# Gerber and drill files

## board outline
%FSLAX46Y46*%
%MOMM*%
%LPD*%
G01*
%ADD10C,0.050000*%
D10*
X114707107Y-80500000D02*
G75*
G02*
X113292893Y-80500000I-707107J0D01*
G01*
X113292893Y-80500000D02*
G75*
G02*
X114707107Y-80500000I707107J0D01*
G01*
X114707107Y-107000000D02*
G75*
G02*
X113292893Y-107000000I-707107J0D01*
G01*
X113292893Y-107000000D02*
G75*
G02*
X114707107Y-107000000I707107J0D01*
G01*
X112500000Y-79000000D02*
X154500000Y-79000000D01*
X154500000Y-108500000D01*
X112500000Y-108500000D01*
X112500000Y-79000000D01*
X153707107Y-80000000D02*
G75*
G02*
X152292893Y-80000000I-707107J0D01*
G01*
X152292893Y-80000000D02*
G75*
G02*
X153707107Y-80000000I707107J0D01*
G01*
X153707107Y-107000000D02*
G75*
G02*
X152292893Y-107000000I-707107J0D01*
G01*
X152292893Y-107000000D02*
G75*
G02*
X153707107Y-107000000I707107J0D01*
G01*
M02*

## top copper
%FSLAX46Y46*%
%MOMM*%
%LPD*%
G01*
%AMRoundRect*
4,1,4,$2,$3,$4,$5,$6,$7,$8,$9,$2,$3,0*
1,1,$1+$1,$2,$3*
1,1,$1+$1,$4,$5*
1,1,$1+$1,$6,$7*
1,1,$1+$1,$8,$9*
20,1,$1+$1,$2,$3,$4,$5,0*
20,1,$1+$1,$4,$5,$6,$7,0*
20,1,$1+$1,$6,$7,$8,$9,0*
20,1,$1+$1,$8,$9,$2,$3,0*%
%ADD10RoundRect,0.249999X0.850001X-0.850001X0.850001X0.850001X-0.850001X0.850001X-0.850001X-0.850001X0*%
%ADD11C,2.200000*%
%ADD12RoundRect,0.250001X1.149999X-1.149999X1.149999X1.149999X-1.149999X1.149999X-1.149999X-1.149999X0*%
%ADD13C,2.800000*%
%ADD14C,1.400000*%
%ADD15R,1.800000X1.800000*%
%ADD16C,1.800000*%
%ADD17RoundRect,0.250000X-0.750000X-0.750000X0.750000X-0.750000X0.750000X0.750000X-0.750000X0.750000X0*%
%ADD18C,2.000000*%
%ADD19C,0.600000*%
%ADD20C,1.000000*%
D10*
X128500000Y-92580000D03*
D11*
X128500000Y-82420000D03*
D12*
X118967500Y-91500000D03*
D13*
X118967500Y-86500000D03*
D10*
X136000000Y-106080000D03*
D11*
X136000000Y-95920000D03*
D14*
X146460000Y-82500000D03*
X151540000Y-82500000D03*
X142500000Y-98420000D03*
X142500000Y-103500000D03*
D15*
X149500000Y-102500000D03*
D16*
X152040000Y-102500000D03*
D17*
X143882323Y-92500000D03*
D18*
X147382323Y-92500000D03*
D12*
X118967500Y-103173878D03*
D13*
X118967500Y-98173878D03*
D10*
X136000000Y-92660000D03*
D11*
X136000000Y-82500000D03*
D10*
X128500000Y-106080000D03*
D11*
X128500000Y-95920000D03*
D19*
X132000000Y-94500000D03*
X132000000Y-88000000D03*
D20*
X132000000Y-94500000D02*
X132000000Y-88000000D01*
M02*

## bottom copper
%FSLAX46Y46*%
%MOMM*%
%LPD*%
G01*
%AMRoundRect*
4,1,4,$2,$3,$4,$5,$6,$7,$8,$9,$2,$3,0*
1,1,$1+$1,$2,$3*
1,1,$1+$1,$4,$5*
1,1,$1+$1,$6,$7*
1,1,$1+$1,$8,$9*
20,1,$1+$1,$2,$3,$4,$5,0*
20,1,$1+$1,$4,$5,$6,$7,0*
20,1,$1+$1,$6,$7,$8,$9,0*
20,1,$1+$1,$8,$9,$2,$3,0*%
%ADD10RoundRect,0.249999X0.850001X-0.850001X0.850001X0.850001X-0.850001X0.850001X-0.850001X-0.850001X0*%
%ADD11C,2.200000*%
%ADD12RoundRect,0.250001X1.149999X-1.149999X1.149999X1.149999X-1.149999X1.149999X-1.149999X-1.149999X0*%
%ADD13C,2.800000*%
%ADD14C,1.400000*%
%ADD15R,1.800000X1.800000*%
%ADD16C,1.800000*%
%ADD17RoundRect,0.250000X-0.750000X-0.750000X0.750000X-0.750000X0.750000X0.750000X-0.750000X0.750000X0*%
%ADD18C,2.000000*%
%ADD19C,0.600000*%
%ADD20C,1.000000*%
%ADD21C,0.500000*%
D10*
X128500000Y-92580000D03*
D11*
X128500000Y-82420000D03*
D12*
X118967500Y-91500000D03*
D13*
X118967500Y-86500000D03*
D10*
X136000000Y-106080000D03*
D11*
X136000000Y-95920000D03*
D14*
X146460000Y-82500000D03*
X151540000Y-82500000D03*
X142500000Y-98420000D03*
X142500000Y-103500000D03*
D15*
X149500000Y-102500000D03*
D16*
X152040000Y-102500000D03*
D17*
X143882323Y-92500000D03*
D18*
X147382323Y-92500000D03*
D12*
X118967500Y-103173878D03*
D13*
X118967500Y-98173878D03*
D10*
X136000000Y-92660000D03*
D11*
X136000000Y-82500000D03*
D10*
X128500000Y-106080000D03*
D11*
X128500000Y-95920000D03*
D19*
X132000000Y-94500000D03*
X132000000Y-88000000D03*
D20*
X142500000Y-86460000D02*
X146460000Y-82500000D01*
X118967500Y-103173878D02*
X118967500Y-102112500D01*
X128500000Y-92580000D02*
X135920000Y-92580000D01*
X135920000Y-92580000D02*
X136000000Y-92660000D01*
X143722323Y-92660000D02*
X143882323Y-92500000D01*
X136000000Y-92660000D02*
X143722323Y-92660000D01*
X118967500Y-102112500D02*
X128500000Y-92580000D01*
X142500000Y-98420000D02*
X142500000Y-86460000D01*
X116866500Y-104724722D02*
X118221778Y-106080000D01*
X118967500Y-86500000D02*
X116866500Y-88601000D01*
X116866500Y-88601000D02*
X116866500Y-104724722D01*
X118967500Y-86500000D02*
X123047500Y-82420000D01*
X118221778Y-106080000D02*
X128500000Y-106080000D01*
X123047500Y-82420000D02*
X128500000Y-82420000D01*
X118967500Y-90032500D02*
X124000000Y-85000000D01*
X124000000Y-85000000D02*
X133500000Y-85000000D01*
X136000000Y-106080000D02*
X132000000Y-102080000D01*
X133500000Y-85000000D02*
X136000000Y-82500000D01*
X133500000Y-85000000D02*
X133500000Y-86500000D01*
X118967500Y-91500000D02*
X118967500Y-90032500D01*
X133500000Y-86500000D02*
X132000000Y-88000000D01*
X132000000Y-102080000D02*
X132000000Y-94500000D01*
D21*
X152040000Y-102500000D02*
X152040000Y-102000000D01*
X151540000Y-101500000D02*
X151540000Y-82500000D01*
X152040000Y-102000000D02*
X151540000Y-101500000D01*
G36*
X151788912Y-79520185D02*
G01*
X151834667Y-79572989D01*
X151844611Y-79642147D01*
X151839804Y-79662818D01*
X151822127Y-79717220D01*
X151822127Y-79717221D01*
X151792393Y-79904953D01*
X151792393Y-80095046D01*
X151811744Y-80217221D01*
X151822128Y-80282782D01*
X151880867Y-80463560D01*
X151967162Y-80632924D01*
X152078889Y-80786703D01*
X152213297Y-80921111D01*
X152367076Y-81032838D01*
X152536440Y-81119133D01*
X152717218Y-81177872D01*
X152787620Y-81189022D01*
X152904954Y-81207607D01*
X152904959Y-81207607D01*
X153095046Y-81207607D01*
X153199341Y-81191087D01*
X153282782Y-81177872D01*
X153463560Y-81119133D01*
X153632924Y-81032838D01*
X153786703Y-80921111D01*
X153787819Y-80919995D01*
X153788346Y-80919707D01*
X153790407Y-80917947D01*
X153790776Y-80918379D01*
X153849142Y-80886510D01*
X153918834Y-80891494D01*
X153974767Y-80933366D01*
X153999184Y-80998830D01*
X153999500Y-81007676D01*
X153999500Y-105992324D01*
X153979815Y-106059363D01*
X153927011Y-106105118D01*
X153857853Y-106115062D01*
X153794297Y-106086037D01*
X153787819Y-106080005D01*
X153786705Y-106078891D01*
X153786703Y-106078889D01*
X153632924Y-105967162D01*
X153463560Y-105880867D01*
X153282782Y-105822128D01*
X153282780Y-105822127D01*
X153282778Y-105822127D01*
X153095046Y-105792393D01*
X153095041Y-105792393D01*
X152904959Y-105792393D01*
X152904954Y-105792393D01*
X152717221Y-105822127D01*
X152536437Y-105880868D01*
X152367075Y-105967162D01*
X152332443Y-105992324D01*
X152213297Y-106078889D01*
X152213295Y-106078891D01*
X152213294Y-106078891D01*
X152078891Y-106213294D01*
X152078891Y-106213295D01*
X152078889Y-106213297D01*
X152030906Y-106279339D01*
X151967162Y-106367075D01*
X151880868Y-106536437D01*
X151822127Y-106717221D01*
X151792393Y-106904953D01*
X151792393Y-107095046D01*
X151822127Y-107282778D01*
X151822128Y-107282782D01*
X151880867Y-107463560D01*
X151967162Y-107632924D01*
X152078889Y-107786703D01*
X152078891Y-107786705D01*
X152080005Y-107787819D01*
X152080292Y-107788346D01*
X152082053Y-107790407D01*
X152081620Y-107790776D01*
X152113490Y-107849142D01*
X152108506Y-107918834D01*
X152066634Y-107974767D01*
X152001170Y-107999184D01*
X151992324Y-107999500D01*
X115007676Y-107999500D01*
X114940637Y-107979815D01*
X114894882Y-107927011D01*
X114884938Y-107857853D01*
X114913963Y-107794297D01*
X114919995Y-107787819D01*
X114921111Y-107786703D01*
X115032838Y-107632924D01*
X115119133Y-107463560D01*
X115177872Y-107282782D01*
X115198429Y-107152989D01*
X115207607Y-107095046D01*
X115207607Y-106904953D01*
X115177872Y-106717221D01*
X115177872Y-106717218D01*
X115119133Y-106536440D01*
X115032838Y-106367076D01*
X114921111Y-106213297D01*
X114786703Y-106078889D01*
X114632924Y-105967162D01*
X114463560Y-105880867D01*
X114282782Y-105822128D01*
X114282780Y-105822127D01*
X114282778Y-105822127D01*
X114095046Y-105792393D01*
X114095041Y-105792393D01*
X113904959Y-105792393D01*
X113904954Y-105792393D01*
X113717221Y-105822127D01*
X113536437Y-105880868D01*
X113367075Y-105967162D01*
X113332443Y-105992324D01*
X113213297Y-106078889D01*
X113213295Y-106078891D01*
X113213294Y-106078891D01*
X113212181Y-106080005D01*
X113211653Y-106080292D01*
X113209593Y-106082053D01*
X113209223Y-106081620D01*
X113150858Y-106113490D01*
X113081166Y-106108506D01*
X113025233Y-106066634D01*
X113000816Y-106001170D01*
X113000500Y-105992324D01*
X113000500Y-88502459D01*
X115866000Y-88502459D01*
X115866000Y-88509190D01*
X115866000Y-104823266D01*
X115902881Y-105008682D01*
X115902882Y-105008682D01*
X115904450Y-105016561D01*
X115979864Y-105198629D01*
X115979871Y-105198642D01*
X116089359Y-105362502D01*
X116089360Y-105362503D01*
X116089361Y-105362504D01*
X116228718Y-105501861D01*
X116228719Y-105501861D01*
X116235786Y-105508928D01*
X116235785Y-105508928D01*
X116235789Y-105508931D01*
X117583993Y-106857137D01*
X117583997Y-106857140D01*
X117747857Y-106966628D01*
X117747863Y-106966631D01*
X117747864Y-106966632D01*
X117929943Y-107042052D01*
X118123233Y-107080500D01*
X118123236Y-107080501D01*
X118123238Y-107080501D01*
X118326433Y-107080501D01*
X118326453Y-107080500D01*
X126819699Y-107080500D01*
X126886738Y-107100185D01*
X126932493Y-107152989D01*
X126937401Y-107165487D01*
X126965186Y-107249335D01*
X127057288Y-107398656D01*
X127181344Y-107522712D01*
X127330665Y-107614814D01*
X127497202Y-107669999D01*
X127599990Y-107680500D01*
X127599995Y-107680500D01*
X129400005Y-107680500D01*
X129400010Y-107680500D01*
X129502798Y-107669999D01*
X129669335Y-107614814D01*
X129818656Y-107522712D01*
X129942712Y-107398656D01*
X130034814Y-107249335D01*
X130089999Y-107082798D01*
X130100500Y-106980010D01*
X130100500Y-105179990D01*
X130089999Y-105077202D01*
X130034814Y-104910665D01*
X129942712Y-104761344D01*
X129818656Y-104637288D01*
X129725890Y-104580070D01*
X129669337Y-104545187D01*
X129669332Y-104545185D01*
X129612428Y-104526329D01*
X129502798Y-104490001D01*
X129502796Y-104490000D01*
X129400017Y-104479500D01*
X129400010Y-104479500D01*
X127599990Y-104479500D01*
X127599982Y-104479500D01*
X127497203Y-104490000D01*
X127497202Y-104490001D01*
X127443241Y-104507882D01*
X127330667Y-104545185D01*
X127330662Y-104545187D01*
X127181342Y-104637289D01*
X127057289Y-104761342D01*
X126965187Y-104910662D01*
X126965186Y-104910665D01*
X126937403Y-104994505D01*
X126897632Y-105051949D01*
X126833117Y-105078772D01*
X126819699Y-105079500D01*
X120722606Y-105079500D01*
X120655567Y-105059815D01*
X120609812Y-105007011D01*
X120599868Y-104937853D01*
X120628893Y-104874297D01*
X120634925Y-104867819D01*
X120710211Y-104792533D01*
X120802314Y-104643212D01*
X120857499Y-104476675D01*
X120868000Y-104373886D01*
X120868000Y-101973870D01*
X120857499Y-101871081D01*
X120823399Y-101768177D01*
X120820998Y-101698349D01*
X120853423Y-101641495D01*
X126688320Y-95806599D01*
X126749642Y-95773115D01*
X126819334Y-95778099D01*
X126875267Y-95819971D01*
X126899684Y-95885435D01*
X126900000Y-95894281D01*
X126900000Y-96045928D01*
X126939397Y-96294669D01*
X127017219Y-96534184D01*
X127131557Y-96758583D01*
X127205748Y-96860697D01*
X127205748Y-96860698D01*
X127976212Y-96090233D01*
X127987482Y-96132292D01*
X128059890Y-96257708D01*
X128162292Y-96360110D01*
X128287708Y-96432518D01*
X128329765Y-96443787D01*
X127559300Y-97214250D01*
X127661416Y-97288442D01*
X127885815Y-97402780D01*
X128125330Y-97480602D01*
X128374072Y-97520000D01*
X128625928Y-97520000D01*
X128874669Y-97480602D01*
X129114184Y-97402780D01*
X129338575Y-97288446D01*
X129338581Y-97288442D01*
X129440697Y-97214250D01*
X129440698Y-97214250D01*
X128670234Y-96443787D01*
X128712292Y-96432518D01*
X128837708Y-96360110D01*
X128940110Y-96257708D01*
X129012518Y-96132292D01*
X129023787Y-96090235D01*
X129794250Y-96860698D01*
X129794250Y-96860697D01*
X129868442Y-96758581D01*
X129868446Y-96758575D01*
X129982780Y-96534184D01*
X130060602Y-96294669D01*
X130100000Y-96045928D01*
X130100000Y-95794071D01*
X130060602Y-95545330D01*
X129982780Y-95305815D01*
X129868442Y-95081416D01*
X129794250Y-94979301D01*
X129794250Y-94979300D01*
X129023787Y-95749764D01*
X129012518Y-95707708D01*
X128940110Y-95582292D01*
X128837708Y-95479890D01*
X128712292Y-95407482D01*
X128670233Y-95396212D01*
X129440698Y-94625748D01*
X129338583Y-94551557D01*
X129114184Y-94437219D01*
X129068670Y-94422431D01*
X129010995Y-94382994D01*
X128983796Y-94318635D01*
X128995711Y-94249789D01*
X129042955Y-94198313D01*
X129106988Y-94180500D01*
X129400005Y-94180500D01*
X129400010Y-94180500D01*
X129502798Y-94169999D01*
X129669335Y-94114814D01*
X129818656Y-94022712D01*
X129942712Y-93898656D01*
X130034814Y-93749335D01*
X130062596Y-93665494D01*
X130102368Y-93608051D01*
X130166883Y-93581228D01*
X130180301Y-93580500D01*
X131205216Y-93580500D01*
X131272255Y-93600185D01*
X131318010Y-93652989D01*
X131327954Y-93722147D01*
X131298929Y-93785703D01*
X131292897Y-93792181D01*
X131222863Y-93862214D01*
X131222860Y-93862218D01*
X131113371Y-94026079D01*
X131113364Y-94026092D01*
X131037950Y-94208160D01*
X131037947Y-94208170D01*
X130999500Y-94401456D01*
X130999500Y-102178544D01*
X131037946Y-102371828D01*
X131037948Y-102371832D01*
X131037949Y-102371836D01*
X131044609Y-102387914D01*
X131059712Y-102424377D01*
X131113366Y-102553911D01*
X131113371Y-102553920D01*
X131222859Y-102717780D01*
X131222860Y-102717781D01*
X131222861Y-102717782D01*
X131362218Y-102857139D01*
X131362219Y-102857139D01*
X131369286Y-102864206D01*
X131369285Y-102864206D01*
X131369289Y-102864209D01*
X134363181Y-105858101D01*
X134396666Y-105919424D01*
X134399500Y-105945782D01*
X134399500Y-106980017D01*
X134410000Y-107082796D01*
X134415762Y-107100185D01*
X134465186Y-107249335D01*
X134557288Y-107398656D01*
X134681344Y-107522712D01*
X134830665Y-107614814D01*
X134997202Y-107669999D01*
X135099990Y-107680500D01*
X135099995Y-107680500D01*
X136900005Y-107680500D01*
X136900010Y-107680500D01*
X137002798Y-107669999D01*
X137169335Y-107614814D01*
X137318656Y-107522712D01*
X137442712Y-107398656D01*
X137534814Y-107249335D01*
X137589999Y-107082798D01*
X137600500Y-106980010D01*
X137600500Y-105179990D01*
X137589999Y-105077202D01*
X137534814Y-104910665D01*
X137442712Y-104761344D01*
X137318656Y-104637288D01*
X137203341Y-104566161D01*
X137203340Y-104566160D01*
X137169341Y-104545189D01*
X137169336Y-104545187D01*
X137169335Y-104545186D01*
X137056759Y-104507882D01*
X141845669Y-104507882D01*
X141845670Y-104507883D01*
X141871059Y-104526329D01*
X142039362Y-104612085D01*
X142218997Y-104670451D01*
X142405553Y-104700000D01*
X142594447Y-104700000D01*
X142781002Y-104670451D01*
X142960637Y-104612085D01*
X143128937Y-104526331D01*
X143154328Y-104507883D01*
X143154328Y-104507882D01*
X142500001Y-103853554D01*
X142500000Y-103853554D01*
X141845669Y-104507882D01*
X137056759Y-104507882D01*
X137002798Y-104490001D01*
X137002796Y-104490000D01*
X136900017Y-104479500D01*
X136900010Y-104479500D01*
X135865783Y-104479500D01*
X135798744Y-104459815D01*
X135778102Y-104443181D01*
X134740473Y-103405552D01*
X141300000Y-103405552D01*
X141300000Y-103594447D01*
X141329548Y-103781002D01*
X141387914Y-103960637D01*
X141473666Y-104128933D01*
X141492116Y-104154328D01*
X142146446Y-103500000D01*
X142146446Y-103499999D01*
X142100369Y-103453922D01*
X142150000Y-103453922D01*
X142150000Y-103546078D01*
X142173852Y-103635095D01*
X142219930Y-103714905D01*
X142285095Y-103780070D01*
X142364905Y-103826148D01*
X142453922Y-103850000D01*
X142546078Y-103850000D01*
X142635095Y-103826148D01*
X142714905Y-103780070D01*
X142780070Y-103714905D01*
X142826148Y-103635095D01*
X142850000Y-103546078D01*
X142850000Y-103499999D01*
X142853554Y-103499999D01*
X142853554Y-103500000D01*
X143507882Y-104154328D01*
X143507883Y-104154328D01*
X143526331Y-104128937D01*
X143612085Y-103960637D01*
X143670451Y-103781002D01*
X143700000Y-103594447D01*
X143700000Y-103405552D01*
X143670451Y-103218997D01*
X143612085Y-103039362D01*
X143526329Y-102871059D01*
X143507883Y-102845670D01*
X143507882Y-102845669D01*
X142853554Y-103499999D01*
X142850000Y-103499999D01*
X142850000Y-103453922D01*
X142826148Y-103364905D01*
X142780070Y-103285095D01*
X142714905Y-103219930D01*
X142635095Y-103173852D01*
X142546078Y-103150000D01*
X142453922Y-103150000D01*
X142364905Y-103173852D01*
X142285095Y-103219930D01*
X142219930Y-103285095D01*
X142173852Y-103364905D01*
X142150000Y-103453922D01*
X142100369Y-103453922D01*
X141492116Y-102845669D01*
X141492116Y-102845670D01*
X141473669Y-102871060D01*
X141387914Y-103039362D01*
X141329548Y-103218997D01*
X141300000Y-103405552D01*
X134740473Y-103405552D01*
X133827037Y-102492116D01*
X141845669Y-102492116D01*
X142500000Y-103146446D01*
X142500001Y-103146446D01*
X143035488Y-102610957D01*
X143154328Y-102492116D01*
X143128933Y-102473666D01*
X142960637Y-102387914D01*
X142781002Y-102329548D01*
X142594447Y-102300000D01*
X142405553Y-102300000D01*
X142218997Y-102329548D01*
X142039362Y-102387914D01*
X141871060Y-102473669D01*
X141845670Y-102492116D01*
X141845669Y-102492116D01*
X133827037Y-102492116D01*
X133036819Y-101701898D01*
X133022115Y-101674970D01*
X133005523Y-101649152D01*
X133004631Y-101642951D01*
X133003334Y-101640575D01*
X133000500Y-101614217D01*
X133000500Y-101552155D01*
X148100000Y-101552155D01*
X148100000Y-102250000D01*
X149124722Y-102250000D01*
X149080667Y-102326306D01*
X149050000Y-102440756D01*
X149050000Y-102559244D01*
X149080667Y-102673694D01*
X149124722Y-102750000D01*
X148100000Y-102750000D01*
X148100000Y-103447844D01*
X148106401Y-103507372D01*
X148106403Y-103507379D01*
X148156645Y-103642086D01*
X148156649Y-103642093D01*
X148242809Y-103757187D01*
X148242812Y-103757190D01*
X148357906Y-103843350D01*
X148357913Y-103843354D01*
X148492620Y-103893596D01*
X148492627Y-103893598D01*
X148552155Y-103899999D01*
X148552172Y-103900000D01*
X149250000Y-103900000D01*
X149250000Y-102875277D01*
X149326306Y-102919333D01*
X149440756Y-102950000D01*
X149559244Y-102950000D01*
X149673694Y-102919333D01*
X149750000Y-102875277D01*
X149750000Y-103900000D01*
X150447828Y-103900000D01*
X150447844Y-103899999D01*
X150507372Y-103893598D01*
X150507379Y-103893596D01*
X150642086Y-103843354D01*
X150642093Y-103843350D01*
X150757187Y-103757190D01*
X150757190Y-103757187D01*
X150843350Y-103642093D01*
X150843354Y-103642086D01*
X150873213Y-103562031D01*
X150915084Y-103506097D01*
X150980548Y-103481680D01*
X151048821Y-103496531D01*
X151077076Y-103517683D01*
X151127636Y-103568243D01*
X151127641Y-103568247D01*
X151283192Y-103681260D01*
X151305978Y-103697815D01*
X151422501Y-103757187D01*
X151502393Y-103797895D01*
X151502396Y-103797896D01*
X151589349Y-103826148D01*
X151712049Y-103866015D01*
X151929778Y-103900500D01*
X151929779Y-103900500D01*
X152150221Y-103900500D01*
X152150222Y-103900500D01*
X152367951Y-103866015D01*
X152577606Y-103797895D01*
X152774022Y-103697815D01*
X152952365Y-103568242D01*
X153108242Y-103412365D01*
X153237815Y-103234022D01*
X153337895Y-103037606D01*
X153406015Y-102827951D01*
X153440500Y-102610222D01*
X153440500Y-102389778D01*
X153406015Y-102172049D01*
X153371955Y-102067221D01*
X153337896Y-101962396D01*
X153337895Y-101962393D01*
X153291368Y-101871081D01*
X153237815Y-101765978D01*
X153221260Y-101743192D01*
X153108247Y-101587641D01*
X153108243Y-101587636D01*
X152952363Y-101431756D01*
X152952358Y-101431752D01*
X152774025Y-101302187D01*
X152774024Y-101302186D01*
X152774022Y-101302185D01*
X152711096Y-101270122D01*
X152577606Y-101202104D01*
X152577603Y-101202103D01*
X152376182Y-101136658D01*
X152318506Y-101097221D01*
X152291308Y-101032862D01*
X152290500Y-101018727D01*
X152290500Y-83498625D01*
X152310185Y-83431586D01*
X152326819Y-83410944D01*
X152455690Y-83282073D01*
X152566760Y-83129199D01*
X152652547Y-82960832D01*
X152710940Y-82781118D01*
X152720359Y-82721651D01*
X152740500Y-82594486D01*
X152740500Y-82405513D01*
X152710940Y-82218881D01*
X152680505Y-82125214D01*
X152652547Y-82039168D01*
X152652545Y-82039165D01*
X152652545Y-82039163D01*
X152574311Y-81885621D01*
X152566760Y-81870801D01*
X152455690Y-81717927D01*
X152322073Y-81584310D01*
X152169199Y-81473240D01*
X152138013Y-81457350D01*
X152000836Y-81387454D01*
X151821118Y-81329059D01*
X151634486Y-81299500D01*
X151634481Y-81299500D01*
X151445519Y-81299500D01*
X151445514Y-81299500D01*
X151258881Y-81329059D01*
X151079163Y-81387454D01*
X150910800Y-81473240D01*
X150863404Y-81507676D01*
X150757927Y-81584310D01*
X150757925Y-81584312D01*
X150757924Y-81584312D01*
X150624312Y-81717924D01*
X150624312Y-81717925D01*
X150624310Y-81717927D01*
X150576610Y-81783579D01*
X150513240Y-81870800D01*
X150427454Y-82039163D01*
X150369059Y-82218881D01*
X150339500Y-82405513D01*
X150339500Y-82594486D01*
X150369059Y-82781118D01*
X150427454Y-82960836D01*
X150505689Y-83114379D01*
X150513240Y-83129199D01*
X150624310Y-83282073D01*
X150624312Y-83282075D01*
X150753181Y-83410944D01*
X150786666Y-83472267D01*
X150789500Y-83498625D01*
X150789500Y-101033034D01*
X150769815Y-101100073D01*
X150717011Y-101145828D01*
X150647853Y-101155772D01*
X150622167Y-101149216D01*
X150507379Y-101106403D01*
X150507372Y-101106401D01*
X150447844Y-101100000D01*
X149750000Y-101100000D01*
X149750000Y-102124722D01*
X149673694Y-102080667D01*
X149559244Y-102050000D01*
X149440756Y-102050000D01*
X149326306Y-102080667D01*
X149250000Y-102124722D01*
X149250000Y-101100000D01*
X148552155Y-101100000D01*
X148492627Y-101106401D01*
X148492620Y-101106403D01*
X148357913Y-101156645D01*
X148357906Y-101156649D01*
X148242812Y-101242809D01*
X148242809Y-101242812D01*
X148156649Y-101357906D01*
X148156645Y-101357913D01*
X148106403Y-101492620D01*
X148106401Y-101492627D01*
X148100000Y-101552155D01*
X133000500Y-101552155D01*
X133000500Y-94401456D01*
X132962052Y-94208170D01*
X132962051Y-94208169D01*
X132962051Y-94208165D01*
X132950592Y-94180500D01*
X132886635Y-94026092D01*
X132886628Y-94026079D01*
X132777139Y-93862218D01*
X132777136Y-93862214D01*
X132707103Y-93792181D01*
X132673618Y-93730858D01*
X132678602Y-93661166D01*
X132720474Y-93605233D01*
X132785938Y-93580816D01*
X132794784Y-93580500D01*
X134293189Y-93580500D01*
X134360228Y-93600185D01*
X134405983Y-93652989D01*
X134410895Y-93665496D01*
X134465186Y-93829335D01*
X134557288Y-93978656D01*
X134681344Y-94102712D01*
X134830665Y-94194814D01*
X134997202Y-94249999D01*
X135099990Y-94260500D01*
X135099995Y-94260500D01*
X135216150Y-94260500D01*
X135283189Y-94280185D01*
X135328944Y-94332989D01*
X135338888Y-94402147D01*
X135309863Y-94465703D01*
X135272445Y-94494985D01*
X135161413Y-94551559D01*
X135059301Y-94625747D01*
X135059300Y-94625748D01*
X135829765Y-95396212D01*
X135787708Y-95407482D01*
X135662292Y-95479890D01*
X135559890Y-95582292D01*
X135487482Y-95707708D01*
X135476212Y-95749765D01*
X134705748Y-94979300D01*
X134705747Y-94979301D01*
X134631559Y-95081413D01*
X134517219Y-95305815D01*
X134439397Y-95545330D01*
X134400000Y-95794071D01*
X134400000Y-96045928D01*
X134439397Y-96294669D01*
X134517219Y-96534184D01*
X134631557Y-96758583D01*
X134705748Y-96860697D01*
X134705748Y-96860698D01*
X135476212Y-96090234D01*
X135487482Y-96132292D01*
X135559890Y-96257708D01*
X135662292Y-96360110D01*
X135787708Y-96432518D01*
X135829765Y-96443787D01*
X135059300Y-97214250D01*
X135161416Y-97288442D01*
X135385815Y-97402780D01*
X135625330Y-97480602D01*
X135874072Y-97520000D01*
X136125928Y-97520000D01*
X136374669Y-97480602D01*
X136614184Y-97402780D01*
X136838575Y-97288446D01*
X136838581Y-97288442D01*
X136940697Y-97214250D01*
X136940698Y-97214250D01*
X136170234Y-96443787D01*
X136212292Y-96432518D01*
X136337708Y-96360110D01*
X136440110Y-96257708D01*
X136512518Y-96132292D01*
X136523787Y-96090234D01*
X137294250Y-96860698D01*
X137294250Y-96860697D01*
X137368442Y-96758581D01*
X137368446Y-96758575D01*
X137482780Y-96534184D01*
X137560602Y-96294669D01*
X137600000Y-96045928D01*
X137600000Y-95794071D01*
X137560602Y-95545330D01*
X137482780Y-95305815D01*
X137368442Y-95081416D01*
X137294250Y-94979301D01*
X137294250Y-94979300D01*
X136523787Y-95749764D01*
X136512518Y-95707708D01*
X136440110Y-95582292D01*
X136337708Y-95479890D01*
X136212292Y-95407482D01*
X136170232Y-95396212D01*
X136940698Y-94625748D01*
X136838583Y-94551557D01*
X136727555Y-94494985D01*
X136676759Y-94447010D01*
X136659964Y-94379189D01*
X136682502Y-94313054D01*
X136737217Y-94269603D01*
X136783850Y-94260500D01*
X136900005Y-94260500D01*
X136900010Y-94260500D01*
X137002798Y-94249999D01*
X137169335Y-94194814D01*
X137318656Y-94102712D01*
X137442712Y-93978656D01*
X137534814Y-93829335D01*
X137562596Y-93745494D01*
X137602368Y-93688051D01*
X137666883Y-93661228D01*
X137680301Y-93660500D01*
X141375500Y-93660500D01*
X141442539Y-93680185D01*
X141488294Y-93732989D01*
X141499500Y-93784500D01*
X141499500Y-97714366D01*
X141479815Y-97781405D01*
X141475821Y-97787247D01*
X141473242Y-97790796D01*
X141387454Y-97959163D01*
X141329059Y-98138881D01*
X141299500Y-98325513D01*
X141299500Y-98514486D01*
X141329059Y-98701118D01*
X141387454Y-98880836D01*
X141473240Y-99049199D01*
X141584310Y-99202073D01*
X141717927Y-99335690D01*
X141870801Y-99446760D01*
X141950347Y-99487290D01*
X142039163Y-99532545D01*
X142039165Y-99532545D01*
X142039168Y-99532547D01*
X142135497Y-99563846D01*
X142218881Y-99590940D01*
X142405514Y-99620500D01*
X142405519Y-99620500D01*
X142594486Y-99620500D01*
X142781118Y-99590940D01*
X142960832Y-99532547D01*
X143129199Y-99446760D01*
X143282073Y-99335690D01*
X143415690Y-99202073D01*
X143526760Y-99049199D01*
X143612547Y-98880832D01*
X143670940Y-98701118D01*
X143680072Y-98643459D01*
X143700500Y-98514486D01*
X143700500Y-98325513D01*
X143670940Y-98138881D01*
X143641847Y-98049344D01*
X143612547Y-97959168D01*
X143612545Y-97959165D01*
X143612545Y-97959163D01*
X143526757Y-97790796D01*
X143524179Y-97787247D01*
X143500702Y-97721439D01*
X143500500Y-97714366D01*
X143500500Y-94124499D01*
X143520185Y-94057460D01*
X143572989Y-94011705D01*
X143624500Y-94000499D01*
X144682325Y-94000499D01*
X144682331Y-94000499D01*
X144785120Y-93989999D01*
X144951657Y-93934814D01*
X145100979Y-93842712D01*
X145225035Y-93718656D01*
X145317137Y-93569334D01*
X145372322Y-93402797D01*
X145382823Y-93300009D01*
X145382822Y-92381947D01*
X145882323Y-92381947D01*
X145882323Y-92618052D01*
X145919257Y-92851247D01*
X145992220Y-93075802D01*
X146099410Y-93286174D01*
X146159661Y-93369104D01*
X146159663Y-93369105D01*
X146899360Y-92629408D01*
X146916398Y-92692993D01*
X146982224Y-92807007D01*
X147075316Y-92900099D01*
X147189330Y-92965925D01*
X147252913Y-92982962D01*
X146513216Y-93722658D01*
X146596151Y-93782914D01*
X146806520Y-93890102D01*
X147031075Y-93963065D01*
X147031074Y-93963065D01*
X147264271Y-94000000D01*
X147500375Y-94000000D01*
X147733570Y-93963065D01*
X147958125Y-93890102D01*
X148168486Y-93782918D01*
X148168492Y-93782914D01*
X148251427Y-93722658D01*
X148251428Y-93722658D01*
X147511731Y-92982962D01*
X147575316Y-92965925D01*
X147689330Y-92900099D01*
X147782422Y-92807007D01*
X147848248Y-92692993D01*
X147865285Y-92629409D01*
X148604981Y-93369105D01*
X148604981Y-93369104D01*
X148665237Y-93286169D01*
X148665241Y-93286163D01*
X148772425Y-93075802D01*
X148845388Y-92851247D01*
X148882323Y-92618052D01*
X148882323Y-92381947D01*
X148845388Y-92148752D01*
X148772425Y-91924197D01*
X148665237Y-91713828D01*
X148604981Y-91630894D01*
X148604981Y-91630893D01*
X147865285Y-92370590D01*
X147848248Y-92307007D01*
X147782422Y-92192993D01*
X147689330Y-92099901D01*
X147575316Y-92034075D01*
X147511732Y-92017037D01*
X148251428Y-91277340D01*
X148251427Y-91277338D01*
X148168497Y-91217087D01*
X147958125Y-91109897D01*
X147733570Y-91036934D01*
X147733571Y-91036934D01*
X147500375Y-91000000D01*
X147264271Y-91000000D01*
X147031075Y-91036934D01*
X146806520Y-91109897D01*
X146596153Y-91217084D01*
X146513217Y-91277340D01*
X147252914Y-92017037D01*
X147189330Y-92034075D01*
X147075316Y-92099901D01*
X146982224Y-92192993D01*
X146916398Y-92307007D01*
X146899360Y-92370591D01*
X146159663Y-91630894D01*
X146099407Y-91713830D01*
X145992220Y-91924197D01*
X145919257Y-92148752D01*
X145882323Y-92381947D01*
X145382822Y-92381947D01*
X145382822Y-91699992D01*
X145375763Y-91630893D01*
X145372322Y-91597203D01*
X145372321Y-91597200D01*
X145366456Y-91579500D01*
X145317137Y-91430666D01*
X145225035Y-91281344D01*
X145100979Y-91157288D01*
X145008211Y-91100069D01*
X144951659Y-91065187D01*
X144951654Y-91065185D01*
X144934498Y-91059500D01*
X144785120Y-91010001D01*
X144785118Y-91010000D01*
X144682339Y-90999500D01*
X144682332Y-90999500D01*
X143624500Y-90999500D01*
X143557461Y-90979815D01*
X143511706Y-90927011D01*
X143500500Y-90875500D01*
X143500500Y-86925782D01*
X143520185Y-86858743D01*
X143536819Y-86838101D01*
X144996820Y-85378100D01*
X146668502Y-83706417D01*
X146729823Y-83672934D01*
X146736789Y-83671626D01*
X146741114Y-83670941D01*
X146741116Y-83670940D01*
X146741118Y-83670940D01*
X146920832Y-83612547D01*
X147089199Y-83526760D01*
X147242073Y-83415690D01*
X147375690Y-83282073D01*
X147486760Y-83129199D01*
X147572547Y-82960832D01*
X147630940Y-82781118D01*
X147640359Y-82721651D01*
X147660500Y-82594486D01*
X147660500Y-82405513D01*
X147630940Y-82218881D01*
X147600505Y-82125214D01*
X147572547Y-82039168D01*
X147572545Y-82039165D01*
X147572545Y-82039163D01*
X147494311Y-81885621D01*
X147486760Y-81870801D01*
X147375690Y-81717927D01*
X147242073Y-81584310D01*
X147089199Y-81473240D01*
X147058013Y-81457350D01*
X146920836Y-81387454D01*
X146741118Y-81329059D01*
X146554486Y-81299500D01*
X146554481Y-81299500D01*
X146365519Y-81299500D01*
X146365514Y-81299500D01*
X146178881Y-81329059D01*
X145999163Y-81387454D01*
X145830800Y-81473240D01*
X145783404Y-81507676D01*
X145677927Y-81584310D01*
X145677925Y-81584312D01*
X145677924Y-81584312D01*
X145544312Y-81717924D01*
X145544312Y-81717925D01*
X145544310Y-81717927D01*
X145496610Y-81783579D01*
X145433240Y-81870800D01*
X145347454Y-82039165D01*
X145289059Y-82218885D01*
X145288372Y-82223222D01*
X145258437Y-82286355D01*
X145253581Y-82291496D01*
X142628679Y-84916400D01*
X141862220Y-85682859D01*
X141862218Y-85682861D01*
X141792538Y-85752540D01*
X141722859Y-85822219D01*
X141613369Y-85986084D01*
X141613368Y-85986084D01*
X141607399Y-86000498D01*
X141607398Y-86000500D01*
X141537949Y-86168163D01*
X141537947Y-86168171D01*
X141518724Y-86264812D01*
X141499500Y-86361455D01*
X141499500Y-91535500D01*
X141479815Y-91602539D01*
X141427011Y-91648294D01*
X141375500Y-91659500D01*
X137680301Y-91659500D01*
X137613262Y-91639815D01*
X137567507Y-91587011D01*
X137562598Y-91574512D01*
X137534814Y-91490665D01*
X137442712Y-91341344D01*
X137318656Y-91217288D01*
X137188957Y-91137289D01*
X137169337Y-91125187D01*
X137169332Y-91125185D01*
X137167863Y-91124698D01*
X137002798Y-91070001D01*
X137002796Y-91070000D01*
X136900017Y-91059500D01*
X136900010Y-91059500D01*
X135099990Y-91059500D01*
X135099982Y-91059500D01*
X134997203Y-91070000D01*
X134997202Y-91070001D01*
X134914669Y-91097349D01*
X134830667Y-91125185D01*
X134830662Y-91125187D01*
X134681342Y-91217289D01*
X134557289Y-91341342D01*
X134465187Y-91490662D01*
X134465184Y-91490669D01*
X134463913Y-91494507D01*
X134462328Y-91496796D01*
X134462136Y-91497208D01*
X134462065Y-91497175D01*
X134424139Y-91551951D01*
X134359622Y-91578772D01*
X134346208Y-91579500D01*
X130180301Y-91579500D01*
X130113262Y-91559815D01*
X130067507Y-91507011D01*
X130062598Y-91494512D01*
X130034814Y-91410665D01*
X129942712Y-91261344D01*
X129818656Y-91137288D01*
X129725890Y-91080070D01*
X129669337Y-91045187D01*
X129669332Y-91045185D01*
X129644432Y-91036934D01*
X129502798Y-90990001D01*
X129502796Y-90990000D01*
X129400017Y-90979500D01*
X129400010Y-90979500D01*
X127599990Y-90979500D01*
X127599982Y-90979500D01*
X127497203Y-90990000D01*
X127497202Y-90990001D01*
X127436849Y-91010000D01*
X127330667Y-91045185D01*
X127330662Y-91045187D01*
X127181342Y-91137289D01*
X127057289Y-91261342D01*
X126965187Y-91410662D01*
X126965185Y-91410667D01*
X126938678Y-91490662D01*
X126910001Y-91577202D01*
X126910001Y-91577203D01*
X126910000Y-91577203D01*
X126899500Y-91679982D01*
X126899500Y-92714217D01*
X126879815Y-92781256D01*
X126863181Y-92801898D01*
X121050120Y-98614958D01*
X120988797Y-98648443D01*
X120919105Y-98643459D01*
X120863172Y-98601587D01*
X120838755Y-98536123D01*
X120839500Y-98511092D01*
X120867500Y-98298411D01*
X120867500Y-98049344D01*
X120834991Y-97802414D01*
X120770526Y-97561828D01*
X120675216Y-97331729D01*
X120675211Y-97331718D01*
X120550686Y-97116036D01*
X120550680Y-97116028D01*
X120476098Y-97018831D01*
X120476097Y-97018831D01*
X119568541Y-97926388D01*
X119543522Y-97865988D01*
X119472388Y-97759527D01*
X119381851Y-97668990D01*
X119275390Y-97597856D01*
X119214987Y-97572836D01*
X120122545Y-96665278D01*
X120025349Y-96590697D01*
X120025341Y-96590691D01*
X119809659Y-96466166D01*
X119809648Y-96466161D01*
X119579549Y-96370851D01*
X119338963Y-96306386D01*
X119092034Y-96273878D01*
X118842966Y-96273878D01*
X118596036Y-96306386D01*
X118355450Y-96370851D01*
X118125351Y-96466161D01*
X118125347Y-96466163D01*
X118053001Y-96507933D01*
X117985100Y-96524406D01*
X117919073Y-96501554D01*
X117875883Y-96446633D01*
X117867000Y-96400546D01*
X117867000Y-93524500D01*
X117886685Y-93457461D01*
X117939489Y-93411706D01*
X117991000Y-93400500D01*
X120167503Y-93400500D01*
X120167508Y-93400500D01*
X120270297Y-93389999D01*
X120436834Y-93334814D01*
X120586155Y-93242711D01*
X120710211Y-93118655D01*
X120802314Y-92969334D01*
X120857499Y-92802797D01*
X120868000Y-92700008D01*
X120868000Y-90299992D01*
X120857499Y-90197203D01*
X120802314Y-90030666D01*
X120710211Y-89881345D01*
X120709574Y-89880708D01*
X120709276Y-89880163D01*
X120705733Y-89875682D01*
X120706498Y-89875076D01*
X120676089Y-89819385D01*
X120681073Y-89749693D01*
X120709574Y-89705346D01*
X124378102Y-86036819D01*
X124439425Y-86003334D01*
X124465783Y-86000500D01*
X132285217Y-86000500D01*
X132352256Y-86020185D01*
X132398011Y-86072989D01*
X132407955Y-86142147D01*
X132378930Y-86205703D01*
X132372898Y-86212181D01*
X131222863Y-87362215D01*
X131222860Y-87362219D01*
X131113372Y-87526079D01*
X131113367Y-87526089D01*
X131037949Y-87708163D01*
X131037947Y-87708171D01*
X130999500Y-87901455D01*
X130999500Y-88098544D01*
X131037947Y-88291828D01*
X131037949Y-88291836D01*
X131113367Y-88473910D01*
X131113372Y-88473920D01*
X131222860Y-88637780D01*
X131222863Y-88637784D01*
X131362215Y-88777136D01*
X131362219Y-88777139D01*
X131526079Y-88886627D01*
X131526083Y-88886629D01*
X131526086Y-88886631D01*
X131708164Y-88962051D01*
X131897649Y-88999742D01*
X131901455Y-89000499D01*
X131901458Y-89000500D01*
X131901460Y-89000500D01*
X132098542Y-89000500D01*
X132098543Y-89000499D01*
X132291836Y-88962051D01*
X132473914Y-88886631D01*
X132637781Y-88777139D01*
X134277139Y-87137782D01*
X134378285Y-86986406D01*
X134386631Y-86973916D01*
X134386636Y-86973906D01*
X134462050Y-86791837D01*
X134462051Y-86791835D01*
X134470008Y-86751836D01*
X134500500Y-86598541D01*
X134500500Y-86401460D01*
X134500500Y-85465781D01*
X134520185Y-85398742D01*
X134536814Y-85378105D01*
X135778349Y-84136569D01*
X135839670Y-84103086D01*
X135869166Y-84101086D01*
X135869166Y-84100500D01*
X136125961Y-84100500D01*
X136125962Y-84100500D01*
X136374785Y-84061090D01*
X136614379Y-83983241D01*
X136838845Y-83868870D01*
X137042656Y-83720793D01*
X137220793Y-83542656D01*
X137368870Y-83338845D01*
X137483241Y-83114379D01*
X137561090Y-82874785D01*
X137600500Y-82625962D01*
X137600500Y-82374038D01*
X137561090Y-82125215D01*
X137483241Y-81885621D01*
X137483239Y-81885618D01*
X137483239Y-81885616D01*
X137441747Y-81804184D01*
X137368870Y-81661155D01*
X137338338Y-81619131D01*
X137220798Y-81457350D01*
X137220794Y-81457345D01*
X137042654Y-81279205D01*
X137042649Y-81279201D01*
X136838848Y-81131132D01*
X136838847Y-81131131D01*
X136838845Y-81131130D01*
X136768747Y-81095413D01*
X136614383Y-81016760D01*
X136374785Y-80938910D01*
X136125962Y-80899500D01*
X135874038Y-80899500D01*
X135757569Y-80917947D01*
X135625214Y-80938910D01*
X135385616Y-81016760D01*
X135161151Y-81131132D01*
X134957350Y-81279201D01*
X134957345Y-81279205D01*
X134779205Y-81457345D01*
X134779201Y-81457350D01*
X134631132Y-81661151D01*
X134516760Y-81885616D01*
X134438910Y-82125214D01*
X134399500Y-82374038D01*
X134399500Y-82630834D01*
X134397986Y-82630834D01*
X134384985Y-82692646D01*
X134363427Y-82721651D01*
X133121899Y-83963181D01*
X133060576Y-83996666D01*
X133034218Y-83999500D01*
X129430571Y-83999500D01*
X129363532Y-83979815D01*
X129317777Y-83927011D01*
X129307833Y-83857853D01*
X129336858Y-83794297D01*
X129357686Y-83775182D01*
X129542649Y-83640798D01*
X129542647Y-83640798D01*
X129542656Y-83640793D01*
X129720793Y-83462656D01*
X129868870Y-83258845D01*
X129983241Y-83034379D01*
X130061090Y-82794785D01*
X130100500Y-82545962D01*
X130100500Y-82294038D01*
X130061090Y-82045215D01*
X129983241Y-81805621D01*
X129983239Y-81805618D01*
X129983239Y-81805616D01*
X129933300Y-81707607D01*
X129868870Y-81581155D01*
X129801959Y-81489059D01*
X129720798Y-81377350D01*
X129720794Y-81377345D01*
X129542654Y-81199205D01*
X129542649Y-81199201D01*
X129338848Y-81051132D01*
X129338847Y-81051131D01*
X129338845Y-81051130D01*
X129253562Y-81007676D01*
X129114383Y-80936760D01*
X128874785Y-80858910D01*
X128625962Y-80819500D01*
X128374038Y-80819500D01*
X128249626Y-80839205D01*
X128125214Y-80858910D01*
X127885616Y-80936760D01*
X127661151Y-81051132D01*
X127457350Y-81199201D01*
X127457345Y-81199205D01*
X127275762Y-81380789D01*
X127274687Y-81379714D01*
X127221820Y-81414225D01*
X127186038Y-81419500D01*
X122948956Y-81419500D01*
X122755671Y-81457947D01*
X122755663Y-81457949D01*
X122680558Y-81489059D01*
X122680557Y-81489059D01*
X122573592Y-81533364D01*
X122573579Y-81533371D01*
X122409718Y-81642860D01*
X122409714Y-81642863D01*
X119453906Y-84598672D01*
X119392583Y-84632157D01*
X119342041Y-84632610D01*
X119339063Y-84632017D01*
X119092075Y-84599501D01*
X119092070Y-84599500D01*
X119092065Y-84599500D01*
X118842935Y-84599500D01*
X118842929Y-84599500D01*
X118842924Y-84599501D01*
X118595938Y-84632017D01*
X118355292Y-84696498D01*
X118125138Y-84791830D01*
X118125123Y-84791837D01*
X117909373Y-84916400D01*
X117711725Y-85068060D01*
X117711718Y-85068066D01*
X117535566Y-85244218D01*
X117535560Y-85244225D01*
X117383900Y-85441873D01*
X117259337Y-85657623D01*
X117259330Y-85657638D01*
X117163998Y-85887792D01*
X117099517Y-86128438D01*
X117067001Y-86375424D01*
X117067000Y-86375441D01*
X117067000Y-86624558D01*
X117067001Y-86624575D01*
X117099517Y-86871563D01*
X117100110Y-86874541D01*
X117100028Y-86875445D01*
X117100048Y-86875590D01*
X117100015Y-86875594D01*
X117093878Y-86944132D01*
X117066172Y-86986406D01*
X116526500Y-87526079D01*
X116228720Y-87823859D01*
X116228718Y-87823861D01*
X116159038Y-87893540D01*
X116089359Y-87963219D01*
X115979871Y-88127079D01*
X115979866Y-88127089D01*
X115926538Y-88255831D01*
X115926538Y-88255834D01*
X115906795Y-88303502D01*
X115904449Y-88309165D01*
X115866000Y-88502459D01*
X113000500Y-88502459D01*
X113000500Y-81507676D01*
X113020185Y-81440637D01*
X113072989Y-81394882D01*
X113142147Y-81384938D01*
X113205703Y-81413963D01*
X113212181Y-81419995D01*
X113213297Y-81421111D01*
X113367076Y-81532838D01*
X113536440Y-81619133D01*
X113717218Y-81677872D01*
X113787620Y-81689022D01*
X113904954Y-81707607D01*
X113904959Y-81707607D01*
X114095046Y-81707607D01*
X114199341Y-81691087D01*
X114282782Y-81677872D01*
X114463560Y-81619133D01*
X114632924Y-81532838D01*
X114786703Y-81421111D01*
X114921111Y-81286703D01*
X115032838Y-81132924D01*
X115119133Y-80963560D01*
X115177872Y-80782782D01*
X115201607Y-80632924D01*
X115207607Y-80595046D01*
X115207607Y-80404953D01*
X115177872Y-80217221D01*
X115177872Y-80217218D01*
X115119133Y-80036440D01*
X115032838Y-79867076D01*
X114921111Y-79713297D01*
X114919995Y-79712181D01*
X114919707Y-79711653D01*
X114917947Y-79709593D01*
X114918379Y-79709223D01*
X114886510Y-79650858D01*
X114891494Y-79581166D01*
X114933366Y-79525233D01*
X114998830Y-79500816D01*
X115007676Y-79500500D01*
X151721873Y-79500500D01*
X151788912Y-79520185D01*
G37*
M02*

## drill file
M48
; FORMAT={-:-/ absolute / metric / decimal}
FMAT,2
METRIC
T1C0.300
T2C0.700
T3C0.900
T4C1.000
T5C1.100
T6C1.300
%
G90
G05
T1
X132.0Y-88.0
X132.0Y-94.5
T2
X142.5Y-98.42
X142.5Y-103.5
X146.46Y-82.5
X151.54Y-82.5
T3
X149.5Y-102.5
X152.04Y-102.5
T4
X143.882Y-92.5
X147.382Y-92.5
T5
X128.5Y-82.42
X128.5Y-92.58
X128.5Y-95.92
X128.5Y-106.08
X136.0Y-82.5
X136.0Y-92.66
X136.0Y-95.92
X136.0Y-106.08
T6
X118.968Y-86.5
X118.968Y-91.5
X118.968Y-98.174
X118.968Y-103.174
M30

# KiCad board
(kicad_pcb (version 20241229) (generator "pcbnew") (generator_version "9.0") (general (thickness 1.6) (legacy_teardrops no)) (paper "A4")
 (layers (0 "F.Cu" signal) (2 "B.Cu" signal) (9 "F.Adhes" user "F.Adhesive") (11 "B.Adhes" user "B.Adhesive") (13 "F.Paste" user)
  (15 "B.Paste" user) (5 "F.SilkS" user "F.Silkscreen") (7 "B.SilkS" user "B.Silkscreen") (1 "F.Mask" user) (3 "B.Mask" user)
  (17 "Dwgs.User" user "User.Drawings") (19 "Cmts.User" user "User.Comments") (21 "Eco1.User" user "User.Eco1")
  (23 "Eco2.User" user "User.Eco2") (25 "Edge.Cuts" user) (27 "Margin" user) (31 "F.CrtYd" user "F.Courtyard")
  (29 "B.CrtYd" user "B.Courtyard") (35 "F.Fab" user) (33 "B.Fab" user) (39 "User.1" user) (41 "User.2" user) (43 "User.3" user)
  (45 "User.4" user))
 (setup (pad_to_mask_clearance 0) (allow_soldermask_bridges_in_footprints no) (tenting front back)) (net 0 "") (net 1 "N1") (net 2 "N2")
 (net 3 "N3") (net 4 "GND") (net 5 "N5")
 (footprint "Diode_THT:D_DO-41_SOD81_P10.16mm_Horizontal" (layer "F.Cu") (at 128.5 92.58 90)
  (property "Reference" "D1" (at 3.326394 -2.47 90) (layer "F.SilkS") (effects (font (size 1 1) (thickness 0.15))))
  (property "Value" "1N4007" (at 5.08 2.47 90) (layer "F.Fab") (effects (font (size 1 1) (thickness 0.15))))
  (pad "1" thru_hole roundrect (at 0 0 90) (size 2.2 2.2) (drill 1.1) (layers "*.Cu" "*.Mask") (remove_unused_layers no)
   (roundrect_rratio 0.113636) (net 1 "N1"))
  (pad "2" thru_hole circle (at 10.16 0 90) (size 2.2 2.2) (drill 1.1) (layers "*.Cu" "*.Mask") (remove_unused_layers no) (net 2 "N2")))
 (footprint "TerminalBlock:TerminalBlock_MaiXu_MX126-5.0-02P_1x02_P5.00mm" (layer "F.Cu") (at 118.9675 91.5 90)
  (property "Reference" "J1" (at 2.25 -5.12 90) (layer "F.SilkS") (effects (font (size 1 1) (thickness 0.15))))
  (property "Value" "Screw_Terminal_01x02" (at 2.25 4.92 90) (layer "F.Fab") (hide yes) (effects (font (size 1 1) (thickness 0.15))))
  (pad "1" thru_hole roundrect (at 0 0 90) (size 2.8 2.8) (drill 1.3) (layers "*.Cu" "*.Mask") (remove_unused_layers no)
   (roundrect_rratio 0.089286) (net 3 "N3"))
  (pad "2" thru_hole circle (at 5 0 90) (size 2.8 2.8) (drill 1.3) (layers "*.Cu" "*.Mask") (remove_unused_layers no) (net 2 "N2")))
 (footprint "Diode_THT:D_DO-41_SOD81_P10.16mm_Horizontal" (layer "F.Cu") (at 136 106.08 90)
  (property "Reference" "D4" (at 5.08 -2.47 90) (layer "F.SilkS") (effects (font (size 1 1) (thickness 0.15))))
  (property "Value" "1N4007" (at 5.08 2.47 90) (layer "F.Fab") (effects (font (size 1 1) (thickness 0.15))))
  (pad "1" thru_hole roundrect (at 0 0 90) (size 2.2 2.2) (drill 1.1) (layers "*.Cu" "*.Mask") (remove_unused_layers no)
   (roundrect_rratio 0.113636) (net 3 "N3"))
  (pad "2" thru_hole circle (at 10.16 0 90) (size 2.2 2.2) (drill 1.1) (layers "*.Cu" "*.Mask") (remove_unused_layers no) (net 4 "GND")))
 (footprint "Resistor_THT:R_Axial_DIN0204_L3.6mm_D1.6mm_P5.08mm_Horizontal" (layer "F.Cu") (at 146.46 82.5)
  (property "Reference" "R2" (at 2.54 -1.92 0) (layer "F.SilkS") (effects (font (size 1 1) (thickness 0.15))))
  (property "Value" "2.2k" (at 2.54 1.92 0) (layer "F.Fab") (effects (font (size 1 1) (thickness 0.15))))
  (pad "1" thru_hole circle (at 0 0) (size 1.4 1.4) (drill 0.7) (layers "*.Cu" "*.Mask") (remove_unused_layers no) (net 1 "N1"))
  (pad "2" thru_hole circle (at 5.08 0) (size 1.4 1.4) (drill 0.7) (layers "*.Cu" "*.Mask") (remove_unused_layers no) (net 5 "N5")))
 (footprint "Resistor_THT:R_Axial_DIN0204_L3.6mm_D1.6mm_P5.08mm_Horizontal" (layer "F.Cu") (at 142.5 98.42 -90)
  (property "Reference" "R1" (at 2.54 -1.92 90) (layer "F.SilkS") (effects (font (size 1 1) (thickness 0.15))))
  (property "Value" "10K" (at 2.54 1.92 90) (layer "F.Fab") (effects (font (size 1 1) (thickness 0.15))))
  (pad "1" thru_hole circle (at 0 0 270) (size 1.4 1.4) (drill 0.7) (layers "*.Cu" "*.Mask") (remove_unused_layers no) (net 1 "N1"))
  (pad "2" thru_hole circle (at 5.08 0 270) (size 1.4 1.4) (drill 0.7) (layers "*.Cu" "*.Mask") (remove_unused_layers no) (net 4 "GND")))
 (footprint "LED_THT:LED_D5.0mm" (layer "F.Cu") (at 149.5 102.5)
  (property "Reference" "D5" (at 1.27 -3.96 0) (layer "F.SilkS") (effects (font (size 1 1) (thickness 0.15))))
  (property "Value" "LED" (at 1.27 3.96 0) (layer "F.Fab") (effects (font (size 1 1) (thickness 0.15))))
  (pad "1" thru_hole rect (at 0 0) (size 1.8 1.8) (drill 0.9) (layers "*.Cu" "*.Mask") (remove_unused_layers no) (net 4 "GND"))
  (pad "2" thru_hole circle (at 2.54 0) (size 1.8 1.8) (drill 0.9) (layers "*.Cu" "*.Mask") (remove_unused_layers no) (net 5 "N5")))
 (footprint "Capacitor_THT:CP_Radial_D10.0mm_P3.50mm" (layer "F.Cu") (at 143.882323 92.5)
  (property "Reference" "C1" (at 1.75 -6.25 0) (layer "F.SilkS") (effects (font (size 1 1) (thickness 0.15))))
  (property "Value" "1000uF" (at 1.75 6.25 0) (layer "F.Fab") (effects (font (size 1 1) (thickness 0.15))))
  (pad "1" thru_hole roundrect (at 0 0) (size 2 2) (drill 1) (layers "*.Cu" "*.Mask") (remove_unused_layers no) (roundrect_rratio 0.125)
   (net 1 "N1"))
  (pad "2" thru_hole circle (at 3.5 0) (size 2 2) (drill 1) (layers "*.Cu" "*.Mask") (remove_unused_layers no) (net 4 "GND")))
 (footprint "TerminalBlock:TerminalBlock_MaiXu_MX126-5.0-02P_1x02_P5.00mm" (layer "F.Cu") (at 118.9675 103.173878 90)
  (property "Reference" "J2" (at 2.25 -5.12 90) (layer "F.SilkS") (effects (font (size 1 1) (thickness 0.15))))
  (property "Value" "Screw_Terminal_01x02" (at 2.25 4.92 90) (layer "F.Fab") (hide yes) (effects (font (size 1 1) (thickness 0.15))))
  (pad "1" thru_hole roundrect (at 0 0 90) (size 2.8 2.8) (drill 1.3) (layers "*.Cu" "*.Mask") (remove_unused_layers no)
   (roundrect_rratio 0.089286) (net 1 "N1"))
  (pad "2" thru_hole circle (at 5 0 90) (size 2.8 2.8) (drill 1.3) (layers "*.Cu" "*.Mask") (remove_unused_layers no) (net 4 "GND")))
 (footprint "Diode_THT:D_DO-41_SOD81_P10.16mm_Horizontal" (layer "F.Cu") (at 136 92.66 90)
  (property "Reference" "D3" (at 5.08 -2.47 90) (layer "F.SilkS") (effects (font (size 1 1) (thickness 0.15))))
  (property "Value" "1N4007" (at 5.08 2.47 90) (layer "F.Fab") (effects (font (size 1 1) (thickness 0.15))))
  (pad "1" thru_hole roundrect (at 0 0 90) (size 2.2 2.2) (drill 1.1) (layers "*.Cu" "*.Mask") (remove_unused_layers no)
   (roundrect_rratio 0.113636) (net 1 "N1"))
  (pad "2" thru_hole circle (at 10.16 0 90) (size 2.2 2.2) (drill 1.1) (layers "*.Cu" "*.Mask") (remove_unused_layers no) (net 3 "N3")))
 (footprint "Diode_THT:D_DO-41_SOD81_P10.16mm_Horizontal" (layer "F.Cu") (at 128.5 106.08 90)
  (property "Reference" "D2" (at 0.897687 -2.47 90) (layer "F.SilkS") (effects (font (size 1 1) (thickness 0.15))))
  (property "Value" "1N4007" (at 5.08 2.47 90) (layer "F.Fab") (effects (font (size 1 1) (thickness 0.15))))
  (pad "1" thru_hole roundrect (at 0 0 90) (size 2.2 2.2) (drill 1.1) (layers "*.Cu" "*.Mask") (remove_unused_layers no)
   (roundrect_rratio 0.113636) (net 2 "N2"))
  (pad "2" thru_hole circle (at 10.16 0 90) (size 2.2 2.2) (drill 1.1) (layers "*.Cu" "*.Mask") (remove_unused_layers no) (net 4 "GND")))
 (gr_circle (center 114 80.5) (end 114.5 81) (stroke (width 0.05) (type default)) (fill no) (layer "Edge.Cuts"))
 (gr_circle (center 114 107) (end 114.5 107.5) (stroke (width 0.05) (type default)) (fill no) (layer "Edge.Cuts"))
 (gr_rect (start 112.5 79) (end 154.5 108.5) (stroke (width 0.05) (type default)) (fill no) (layer "Edge.Cuts"))
 (gr_circle (center 153 80) (end 153.5 80.5) (stroke (width 0.05) (type default)) (fill no) (layer "Edge.Cuts"))
 (gr_circle (center 153 107) (end 153.5 107.5) (stroke (width 0.05) (type default)) (fill no) (layer "Edge.Cuts"))
 (segment (start 142.5 86.46) (end 146.46 82.5) (width 1) (layer "B.Cu") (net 1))
 (segment (start 118.9675 103.173878) (end 118.9675 102.1125) (width 1) (layer "B.Cu") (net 1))
 (segment (start 128.5 92.58) (end 135.92 92.58) (width 1) (layer "B.Cu") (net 1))
 (segment (start 135.92 92.58) (end 136 92.66) (width 1) (layer "B.Cu") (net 1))
 (segment (start 143.722323 92.66) (end 143.882323 92.5) (width 1) (layer "B.Cu") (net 1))
 (segment (start 136 92.66) (end 143.722323 92.66) (width 1) (layer "B.Cu") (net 1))
 (segment (start 118.9675 102.1125) (end 128.5 92.58) (width 1) (layer "B.Cu") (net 1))
 (segment (start 142.5 98.42) (end 142.5 86.46) (width 1) (layer "B.Cu") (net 1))
 (segment (start 116.8665 104.724722) (end 118.221778 106.08) (width 1) (layer "B.Cu") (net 2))
 (segment (start 118.9675 86.5) (end 116.8665 88.601) (width 1) (layer "B.Cu") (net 2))
 (segment (start 116.8665 88.601) (end 116.8665 104.724722) (width 1) (layer "B.Cu") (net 2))
 (segment (start 118.9675 86.5) (end 123.0475 82.42) (width 1) (layer "B.Cu") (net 2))
 (segment (start 118.221778 106.08) (end 128.5 106.08) (width 1) (layer "B.Cu") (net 2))
 (segment (start 123.0475 82.42) (end 128.5 82.42) (width 1) (layer "B.Cu") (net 2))
 (segment (start 132 94.5) (end 132 88) (width 1) (layer "F.Cu") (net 3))
 (via (at 132 94.5) (size 0.6) (drill 0.3) (layers "F.Cu" "B.Cu") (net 3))
 (via (at 132 88) (size 0.6) (drill 0.3) (layers "F.Cu" "B.Cu") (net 3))
 (segment (start 118.9675 90.0325) (end 124 85) (width 1) (layer "B.Cu") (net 3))
 (segment (start 124 85) (end 133.5 85) (width 1) (layer "B.Cu") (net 3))
 (segment (start 136 106.08) (end 132 102.08) (width 1) (layer "B.Cu") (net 3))
 (segment (start 133.5 85) (end 136 82.5) (width 1) (layer "B.Cu") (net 3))
 (segment (start 133.5 85) (end 133.5 86.5) (width 1) (layer "B.Cu") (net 3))
 (segment (start 118.9675 91.5) (end 118.9675 90.0325) (width 1) (layer "B.Cu") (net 3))
 (segment (start 133.5 86.5) (end 132 88) (width 1) (layer "B.Cu") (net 3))
 (segment (start 132 102.08) (end 132 94.5) (width 1) (layer "B.Cu") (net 3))
 (segment (start 152.04 102.5) (end 152.04 102) (width 0.5) (layer "B.Cu") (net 5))
 (segment (start 151.54 101.5) (end 151.54 82.5) (width 0.5) (layer "B.Cu") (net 5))
 (segment (start 152.04 102) (end 151.54 101.5) (width 0.5) (layer "B.Cu") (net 5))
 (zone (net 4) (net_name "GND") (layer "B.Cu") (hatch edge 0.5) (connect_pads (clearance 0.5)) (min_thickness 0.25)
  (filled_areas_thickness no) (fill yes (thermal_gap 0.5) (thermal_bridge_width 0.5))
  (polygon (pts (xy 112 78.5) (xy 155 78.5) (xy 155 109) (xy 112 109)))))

